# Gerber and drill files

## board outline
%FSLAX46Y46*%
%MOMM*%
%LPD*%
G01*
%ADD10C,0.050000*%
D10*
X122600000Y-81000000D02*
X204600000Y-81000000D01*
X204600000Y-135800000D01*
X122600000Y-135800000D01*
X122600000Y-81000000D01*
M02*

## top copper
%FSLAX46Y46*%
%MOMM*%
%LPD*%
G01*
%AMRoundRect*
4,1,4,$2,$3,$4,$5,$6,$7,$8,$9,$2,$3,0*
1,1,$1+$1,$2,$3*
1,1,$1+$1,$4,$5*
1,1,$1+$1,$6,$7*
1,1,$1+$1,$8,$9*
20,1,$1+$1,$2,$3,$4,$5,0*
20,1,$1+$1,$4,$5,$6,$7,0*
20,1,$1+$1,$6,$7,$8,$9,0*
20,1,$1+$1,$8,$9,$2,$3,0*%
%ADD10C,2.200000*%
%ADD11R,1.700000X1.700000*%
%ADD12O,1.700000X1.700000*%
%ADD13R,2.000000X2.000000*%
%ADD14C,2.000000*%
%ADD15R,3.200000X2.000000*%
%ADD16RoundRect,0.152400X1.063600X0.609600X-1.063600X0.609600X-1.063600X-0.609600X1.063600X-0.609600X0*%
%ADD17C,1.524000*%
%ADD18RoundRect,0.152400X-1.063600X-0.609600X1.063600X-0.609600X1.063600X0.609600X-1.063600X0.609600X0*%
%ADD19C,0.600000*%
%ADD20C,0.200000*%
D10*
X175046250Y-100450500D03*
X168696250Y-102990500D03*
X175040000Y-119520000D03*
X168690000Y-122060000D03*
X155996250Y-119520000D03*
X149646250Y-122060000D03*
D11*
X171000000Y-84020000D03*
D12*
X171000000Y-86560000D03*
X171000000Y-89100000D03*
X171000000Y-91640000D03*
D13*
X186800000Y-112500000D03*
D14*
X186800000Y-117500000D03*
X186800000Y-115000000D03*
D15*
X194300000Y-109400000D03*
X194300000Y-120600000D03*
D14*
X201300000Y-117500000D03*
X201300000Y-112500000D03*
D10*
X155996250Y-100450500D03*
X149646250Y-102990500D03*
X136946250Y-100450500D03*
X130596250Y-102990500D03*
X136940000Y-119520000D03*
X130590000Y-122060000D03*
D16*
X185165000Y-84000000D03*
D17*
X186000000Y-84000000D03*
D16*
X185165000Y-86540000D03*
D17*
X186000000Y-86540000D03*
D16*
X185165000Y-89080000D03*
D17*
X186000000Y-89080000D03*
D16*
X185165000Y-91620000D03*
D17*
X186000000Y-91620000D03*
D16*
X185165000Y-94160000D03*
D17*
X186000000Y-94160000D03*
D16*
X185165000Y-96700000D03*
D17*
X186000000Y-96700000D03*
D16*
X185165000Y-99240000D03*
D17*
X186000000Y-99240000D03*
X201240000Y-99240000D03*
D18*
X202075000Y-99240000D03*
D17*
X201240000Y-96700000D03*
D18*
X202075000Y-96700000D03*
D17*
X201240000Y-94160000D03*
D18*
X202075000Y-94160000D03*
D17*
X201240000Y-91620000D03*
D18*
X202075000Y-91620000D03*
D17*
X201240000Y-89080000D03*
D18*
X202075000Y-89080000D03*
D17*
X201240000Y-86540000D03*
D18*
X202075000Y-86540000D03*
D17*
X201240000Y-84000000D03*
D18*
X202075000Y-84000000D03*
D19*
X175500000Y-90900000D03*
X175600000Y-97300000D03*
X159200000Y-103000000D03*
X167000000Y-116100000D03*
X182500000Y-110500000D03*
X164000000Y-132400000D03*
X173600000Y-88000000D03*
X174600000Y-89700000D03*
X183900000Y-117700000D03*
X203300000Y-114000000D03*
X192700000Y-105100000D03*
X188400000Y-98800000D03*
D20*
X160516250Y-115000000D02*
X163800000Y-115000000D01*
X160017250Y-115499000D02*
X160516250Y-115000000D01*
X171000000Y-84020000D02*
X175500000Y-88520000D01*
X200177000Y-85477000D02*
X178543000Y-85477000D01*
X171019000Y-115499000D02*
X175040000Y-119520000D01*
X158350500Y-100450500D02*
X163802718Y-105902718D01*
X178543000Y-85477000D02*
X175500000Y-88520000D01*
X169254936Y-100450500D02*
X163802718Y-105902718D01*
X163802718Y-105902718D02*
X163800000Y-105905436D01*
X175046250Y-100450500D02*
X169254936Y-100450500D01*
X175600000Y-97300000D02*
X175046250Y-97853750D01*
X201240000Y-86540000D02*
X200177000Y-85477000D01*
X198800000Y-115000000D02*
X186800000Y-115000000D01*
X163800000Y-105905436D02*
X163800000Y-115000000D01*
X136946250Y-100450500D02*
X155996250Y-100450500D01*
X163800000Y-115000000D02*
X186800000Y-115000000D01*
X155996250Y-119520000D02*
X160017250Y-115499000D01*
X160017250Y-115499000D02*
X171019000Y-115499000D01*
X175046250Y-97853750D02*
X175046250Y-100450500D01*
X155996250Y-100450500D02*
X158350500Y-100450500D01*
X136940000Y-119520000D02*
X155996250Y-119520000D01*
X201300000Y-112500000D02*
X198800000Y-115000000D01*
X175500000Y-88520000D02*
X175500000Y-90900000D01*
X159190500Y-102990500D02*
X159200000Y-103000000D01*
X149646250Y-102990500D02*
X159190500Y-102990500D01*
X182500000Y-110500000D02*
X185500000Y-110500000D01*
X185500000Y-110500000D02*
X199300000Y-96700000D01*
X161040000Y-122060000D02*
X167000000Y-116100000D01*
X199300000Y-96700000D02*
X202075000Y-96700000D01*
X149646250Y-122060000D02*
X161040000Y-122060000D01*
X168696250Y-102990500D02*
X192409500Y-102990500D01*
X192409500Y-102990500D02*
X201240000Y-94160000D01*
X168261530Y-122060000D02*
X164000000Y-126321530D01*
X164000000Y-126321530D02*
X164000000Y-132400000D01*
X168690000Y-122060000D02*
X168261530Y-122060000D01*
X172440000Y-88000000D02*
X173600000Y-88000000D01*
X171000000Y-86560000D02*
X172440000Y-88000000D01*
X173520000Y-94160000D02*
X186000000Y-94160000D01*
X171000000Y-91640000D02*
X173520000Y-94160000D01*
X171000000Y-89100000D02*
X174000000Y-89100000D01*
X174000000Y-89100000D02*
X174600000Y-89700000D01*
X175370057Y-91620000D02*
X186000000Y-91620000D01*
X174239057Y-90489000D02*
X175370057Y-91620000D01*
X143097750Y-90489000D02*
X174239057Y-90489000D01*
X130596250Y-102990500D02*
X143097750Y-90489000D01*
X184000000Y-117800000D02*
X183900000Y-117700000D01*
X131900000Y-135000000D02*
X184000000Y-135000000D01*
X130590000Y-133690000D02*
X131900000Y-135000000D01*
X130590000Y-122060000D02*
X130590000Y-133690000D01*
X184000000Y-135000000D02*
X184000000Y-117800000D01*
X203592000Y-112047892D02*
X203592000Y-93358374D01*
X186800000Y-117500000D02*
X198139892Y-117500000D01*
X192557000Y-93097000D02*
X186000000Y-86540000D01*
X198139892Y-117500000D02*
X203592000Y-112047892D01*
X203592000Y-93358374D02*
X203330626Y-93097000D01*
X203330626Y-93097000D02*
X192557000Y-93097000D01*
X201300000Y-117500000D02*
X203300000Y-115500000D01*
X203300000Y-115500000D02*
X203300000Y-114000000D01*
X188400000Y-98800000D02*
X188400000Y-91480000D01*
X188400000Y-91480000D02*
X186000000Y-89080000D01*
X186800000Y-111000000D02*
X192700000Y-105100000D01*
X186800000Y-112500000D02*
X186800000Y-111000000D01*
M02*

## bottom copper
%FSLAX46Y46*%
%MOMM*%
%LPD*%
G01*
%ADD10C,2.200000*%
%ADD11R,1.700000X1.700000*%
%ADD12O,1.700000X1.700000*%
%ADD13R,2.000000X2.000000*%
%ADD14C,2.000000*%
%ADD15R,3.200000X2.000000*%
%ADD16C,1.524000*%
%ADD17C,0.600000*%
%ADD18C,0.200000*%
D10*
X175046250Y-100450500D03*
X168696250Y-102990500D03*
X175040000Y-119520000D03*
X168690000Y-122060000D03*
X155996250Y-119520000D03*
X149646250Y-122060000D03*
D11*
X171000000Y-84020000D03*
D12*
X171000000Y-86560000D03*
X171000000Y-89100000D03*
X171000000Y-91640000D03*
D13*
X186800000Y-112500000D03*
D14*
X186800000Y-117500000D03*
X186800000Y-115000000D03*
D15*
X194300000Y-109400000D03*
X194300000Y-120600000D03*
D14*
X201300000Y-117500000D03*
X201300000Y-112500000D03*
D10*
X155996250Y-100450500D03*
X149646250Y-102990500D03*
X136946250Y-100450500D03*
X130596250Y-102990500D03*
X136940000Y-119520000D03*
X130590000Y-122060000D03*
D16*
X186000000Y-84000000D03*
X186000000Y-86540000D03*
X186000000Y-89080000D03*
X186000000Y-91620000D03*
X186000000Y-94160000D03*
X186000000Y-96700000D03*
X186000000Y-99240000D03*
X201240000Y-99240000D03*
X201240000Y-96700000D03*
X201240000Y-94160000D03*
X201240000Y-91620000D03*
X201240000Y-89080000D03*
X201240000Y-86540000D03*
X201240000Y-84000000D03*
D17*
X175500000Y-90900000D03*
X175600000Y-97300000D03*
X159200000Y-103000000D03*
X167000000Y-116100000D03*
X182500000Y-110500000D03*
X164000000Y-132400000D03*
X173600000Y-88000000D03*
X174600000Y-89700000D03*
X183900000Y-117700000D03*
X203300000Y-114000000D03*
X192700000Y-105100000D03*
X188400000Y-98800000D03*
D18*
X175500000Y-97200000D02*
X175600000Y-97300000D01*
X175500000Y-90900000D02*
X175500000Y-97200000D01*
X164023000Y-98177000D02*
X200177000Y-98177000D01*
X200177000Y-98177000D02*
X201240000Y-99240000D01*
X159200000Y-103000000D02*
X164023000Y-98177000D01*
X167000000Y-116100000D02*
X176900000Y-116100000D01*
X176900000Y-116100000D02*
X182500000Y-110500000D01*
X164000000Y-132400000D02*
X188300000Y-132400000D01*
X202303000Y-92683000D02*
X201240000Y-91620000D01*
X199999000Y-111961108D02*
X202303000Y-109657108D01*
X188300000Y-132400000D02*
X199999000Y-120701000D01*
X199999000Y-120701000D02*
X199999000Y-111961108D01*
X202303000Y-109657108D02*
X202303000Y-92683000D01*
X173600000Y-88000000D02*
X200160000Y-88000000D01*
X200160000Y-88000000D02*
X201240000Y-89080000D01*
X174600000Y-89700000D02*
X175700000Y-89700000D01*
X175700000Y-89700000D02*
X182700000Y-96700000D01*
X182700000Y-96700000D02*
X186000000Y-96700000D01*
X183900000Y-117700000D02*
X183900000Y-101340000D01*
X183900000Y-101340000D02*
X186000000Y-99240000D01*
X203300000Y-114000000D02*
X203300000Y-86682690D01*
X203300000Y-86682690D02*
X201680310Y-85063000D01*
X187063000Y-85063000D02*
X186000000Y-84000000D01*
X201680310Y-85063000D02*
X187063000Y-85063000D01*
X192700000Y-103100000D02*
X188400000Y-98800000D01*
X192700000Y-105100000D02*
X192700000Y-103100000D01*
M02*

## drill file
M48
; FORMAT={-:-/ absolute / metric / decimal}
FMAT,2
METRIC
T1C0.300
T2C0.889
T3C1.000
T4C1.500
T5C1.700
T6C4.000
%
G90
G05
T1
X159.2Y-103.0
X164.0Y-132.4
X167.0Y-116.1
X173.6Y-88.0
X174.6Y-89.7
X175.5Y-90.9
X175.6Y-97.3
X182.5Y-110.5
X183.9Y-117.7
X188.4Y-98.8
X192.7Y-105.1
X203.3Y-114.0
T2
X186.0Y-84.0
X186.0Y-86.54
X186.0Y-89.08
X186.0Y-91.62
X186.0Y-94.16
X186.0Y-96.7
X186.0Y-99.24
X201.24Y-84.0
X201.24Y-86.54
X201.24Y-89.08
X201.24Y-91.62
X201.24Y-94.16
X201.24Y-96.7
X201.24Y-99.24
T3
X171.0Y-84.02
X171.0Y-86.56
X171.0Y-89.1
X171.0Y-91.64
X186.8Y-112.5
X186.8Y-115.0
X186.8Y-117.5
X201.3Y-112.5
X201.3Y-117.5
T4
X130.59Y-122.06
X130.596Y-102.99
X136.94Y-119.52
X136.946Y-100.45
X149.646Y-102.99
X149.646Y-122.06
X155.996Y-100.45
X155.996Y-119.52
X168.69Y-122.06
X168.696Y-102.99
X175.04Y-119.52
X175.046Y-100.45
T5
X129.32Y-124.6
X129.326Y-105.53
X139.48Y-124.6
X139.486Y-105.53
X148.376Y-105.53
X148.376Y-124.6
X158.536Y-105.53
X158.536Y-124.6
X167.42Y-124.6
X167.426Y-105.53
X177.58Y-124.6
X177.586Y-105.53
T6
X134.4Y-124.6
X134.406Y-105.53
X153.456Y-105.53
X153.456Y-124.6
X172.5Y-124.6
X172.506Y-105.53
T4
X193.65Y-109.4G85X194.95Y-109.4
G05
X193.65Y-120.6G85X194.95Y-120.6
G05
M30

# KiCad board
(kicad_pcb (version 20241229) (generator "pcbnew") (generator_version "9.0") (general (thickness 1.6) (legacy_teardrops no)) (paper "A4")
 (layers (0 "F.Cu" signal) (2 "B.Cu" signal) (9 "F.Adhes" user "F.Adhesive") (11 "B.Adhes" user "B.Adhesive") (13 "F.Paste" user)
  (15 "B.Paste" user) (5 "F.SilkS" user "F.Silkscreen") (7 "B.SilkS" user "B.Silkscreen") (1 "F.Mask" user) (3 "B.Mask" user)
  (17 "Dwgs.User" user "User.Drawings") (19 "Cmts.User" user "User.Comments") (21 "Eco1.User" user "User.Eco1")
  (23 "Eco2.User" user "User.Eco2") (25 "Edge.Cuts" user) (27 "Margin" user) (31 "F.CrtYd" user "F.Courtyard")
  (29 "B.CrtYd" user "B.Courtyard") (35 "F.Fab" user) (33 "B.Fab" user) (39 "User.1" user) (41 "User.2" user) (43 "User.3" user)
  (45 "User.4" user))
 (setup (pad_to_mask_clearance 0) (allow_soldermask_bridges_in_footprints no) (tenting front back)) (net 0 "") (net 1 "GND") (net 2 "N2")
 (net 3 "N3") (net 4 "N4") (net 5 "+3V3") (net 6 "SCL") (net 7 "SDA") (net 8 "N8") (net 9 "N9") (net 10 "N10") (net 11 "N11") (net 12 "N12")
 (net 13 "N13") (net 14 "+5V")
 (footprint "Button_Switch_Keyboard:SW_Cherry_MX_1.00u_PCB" (layer "F.Cu") (at 175.04625 100.4505)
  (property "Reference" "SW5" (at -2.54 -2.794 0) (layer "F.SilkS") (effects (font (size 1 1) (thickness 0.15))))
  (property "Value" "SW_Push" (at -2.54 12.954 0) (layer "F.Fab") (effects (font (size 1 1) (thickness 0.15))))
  (pad "" np_thru_hole circle (at -7.62 5.08) (size 1.7 1.7) (drill 1.7) (layers "*.Cu" "*.Mask"))
  (pad "" np_thru_hole circle (at -2.54 5.08) (size 4 4) (drill 4) (layers "*.Cu" "*.Mask"))
  (pad "" np_thru_hole circle (at 2.54 5.08) (size 1.7 1.7) (drill 1.7) (layers "*.Cu" "*.Mask"))
  (pad "1" thru_hole circle (at 0 0) (size 2.2 2.2) (drill 1.5) (layers "*.Cu" "*.Mask") (remove_unused_layers no) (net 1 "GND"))
  (pad "2" thru_hole circle (at -6.35 2.54) (size 2.2 2.2) (drill 1.5) (layers "*.Cu" "*.Mask") (remove_unused_layers no) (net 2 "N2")))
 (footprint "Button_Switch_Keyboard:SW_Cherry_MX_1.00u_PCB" (layer "F.Cu") (at 175.04 119.52)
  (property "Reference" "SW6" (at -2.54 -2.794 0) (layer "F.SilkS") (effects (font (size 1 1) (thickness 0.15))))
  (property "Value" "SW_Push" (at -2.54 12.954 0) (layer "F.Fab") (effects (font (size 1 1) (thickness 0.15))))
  (pad "" np_thru_hole circle (at -7.62 5.08) (size 1.7 1.7) (drill 1.7) (layers "*.Cu" "*.Mask"))
  (pad "" np_thru_hole circle (at -2.54 5.08) (size 4 4) (drill 4) (layers "*.Cu" "*.Mask"))
  (pad "" np_thru_hole circle (at 2.54 5.08) (size 1.7 1.7) (drill 1.7) (layers "*.Cu" "*.Mask"))
  (pad "1" thru_hole circle (at 0 0) (size 2.2 2.2) (drill 1.5) (layers "*.Cu" "*.Mask") (remove_unused_layers no) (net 1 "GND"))
  (pad "2" thru_hole circle (at -6.35 2.54) (size 2.2 2.2) (drill 1.5) (layers "*.Cu" "*.Mask") (remove_unused_layers no) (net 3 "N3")))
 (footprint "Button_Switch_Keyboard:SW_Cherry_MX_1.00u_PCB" (layer "F.Cu") (at 155.99625 119.52)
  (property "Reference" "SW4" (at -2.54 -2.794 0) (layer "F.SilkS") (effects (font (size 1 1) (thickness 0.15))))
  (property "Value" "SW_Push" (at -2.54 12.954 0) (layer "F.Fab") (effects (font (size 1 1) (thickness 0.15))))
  (pad "" np_thru_hole circle (at -7.62 5.08) (size 1.7 1.7) (drill 1.7) (layers "*.Cu" "*.Mask"))
  (pad "" np_thru_hole circle (at -2.54 5.08) (size 4 4) (drill 4) (layers "*.Cu" "*.Mask"))
  (pad "" np_thru_hole circle (at 2.54 5.08) (size 1.7 1.7) (drill 1.7) (layers "*.Cu" "*.Mask"))
  (pad "1" thru_hole circle (at 0 0) (size 2.2 2.2) (drill 1.5) (layers "*.Cu" "*.Mask") (remove_unused_layers no) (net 1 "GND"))
  (pad "2" thru_hole circle (at -6.35 2.54) (size 2.2 2.2) (drill 1.5) (layers "*.Cu" "*.Mask") (remove_unused_layers no) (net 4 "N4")))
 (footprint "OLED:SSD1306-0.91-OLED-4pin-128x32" (layer "F.Cu") (at 134.5 81.83)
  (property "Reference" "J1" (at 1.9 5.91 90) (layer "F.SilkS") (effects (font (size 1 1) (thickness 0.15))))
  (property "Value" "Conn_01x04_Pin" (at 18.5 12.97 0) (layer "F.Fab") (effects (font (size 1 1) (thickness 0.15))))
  (pad "1" thru_hole rect (at 36.5 2.19) (size 1.7 1.7) (drill 1) (layers "*.Cu" "*.Mask") (remove_unused_layers no) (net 1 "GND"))
  (pad "2" thru_hole oval (at 36.5 4.73) (size 1.7 1.7) (drill 1) (layers "*.Cu" "*.Mask") (remove_unused_layers no) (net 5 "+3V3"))
  (pad "3" thru_hole oval (at 36.5 7.27) (size 1.7 1.7) (drill 1) (layers "*.Cu" "*.Mask") (remove_unused_layers no) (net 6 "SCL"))
  (pad "4" thru_hole oval (at 36.5 9.81) (size 1.7 1.7) (drill 1) (layers "*.Cu" "*.Mask") (remove_unused_layers no) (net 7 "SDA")))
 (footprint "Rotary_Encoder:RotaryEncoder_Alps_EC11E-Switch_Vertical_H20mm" (layer "F.Cu") (at 186.8 112.5)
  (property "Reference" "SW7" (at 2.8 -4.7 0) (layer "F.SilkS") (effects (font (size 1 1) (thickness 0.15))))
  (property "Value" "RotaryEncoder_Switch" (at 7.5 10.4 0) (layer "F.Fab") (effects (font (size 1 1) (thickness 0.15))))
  (pad "A" thru_hole rect (at 0 0) (size 2 2) (drill 1) (layers "*.Cu" "*.Mask") (remove_unused_layers no) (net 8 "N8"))
  (pad "B" thru_hole circle (at 0 5) (size 2 2) (drill 1) (layers "*.Cu" "*.Mask") (remove_unused_layers no) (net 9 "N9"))
  (pad "C" thru_hole circle (at 0 2.5) (size 2 2) (drill 1) (layers "*.Cu" "*.Mask") (remove_unused_layers no) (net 1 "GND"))
  (pad "MP" thru_hole rect (at 7.5 -3.1) (size 3.2 2) (drill oval 2.8 1.5) (layers "*.Cu" "*.Mask") (remove_unused_layers no))
  (pad "MP" thru_hole rect (at 7.5 8.1) (size 3.2 2) (drill oval 2.8 1.5) (layers "*.Cu" "*.Mask") (remove_unused_layers no))
  (pad "S1" thru_hole circle (at 14.5 5) (size 2 2) (drill 1) (layers "*.Cu" "*.Mask") (remove_unused_layers no) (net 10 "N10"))
  (pad "S2" thru_hole circle (at 14.5 0) (size 2 2) (drill 1) (layers "*.Cu" "*.Mask") (remove_unused_layers no) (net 1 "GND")))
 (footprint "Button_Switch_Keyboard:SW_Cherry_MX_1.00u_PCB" (layer "F.Cu") (at 155.99625 100.4505)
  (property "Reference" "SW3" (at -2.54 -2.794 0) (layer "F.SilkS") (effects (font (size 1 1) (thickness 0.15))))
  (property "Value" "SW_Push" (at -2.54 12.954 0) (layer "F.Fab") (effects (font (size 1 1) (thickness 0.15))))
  (pad "" np_thru_hole circle (at -7.62 5.08) (size 1.7 1.7) (drill 1.7) (layers "*.Cu" "*.Mask"))
  (pad "" np_thru_hole circle (at -2.54 5.08) (size 4 4) (drill 4) (layers "*.Cu" "*.Mask"))
  (pad "" np_thru_hole circle (at 2.54 5.08) (size 1.7 1.7) (drill 1.7) (layers "*.Cu" "*.Mask"))
  (pad "1" thru_hole circle (at 0 0) (size 2.2 2.2) (drill 1.5) (layers "*.Cu" "*.Mask") (remove_unused_layers no) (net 1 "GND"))
  (pad "2" thru_hole circle (at -6.35 2.54) (size 2.2 2.2) (drill 1.5) (layers "*.Cu" "*.Mask") (remove_unused_layers no) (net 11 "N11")))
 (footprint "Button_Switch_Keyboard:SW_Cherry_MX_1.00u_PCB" (layer "F.Cu") (at 136.94625 100.4505)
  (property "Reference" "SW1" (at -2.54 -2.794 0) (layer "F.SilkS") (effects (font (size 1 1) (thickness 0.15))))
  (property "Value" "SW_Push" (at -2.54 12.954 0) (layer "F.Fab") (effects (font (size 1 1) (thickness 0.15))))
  (pad "" np_thru_hole circle (at -7.62 5.08) (size 1.7 1.7) (drill 1.7) (layers "*.Cu" "*.Mask"))
  (pad "" np_thru_hole circle (at -2.54 5.08) (size 4 4) (drill 4) (layers "*.Cu" "*.Mask"))
  (pad "" np_thru_hole circle (at 2.54 5.08) (size 1.7 1.7) (drill 1.7) (layers "*.Cu" "*.Mask"))
  (pad "1" thru_hole circle (at 0 0) (size 2.2 2.2) (drill 1.5) (layers "*.Cu" "*.Mask") (remove_unused_layers no) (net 1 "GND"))
  (pad "2" thru_hole circle (at -6.35 2.54) (size 2.2 2.2) (drill 1.5) (layers "*.Cu" "*.Mask") (remove_unused_layers no) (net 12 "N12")))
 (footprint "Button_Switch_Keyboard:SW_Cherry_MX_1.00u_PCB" (layer "F.Cu") (at 136.94 119.52)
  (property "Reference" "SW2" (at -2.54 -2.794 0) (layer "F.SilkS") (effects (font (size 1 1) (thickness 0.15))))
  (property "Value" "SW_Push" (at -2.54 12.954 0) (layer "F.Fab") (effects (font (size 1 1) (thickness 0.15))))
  (pad "" np_thru_hole circle (at -7.62 5.08) (size 1.7 1.7) (drill 1.7) (layers "*.Cu" "*.Mask"))
  (pad "" np_thru_hole circle (at -2.54 5.08) (size 4 4) (drill 4) (layers "*.Cu" "*.Mask"))
  (pad "" np_thru_hole circle (at 2.54 5.08) (size 1.7 1.7) (drill 1.7) (layers "*.Cu" "*.Mask"))
  (pad "1" thru_hole circle (at 0 0) (size 2.2 2.2) (drill 1.5) (layers "*.Cu" "*.Mask") (remove_unused_layers no) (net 1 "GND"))
  (pad "2" thru_hole circle (at -6.35 2.54) (size 2.2 2.2) (drill 1.5) (layers "*.Cu" "*.Mask") (remove_unused_layers no) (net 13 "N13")))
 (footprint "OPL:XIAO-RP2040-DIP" (layer "F.Cu") (at 193.62 91.62)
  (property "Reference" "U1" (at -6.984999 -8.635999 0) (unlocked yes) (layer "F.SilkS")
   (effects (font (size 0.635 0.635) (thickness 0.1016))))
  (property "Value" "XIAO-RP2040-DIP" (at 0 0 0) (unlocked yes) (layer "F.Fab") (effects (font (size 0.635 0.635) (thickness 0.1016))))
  (pad "1" smd roundrect (at -8.455 -7.62 180) (size 2.432 1.524) (layers "F.Cu" "F.Mask") (roundrect_rratio 0.1) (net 10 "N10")
   (thermal_bridge_angle 45))
  (pad "1" thru_hole circle (at -7.62 -7.62 180) (size 1.524 1.524) (drill 0.889) (layers "*.Cu" "*.Mask") (remove_unused_layers no)
   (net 10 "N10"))
  (pad "2" smd roundrect (at -8.455 -5.08 180) (size 2.432 1.524) (layers "F.Cu" "F.Mask") (roundrect_rratio 0.1) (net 9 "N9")
   (thermal_bridge_angle 45))
  (pad "2" thru_hole circle (at -7.62 -5.08 180) (size 1.524 1.524) (drill 0.889) (layers "*.Cu" "*.Mask") (remove_unused_layers no)
   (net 9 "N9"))
  (pad "3" smd roundrect (at -8.455 -2.54 180) (size 2.432 1.524) (layers "F.Cu" "F.Mask") (roundrect_rratio 0.1) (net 8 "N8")
   (thermal_bridge_angle 45))
  (pad "3" thru_hole circle (at -7.62 -2.54 180) (size 1.524 1.524) (drill 0.889) (layers "*.Cu" "*.Mask") (remove_unused_layers no)
   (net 8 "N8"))
  (pad "4" smd roundrect (at -8.455 0 180) (size 2.432 1.524) (layers "F.Cu" "F.Mask") (roundrect_rratio 0.1) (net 12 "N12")
   (thermal_bridge_angle 45))
  (pad "4" thru_hole circle (at -7.62 0 180) (size 1.524 1.524) (drill 0.889) (layers "*.Cu" "*.Mask") (remove_unused_layers no)
   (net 12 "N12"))
  (pad "5" smd roundrect (at -8.455 2.54 180) (size 2.432 1.524) (layers "F.Cu" "F.Mask") (roundrect_rratio 0.1) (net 7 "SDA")
   (thermal_bridge_angle 45))
  (pad "5" thru_hole circle (at -7.62 2.54 180) (size 1.524 1.524) (drill 0.889) (layers "*.Cu" "*.Mask") (remove_unused_layers no)
   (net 7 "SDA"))
  (pad "6" smd roundrect (at -8.455 5.08 180) (size 2.432 1.524) (layers "F.Cu" "F.Mask") (roundrect_rratio 0.1) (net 6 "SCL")
   (thermal_bridge_angle 45))
  (pad "6" thru_hole circle (at -7.62 5.08 180) (size 1.524 1.524) (drill 0.889) (layers "*.Cu" "*.Mask") (remove_unused_layers no)
   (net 6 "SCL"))
  (pad "7" smd roundrect (at -8.455 7.62 180) (size 2.432 1.524) (layers "F.Cu" "F.Mask") (roundrect_rratio 0.1) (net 13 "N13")
   (thermal_bridge_angle 45))
  (pad "7" thru_hole circle (at -7.62 7.62 180) (size 1.524 1.524) (drill 0.889) (layers "*.Cu" "*.Mask") (remove_unused_layers no)
   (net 13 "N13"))
  (pad "8" thru_hole circle (at 7.62 7.62) (size 1.524 1.524) (drill 0.889) (layers "*.Cu" "*.Mask") (remove_unused_layers no)
   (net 11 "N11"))
  (pad "8" smd roundrect (at 8.455 7.62) (size 2.432 1.524) (layers "F.Cu" "F.Mask") (roundrect_rratio 0.1) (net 11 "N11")
   (thermal_bridge_angle 45))
  (pad "9" thru_hole circle (at 7.62 5.08) (size 1.524 1.524) (drill 0.889) (layers "*.Cu" "*.Mask") (remove_unused_layers no) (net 4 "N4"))
  (pad "9" smd roundrect (at 8.455 5.08) (size 2.432 1.524) (layers "F.Cu" "F.Mask") (roundrect_rratio 0.1) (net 4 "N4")
   (thermal_bridge_angle 45))
  (pad "10" thru_hole circle (at 7.62 2.54) (size 1.524 1.524) (drill 0.889) (layers "*.Cu" "*.Mask") (remove_unused_layers no) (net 2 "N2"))
  (pad "10" smd roundrect (at 8.455 2.54) (size 2.432 1.524) (layers "F.Cu" "F.Mask") (roundrect_rratio 0.1) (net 2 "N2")
   (thermal_bridge_angle 45))
  (pad "11" thru_hole circle (at 7.62 0) (size 1.524 1.524) (drill 0.889) (layers "*.Cu" "*.Mask") (remove_unused_layers no) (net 3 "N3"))
  (pad "11" smd roundrect (at 8.455 0) (size 2.432 1.524) (layers "F.Cu" "F.Mask") (roundrect_rratio 0.1) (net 3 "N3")
   (thermal_bridge_angle 45))
  (pad "12" thru_hole circle (at 7.62 -2.54) (size 1.524 1.524) (drill 0.889) (layers "*.Cu" "*.Mask") (remove_unused_layers no)
   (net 5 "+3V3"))
  (pad "12" smd roundrect (at 8.455 -2.54) (size 2.432 1.524) (layers "F.Cu" "F.Mask") (roundrect_rratio 0.1) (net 5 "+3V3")
   (thermal_bridge_angle 45))
  (pad "13" thru_hole circle (at 7.62 -5.08) (size 1.524 1.524) (drill 0.889) (layers "*.Cu" "*.Mask") (remove_unused_layers no)
   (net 1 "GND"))
  (pad "13" smd roundrect (at 8.455 -5.08) (size 2.432 1.524) (layers "F.Cu" "F.Mask") (roundrect_rratio 0.1) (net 1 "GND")
   (thermal_bridge_angle 45))
  (pad "14" thru_hole circle (at 7.62 -7.62) (size 1.524 1.524) (drill 0.889) (layers "*.Cu" "*.Mask") (remove_unused_layers no)
   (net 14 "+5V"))
  (pad "14" smd roundrect (at 8.455 -7.62) (size 2.432 1.524) (layers "F.Cu" "F.Mask") (roundrect_rratio 0.1) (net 14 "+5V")
   (thermal_bridge_angle 45)))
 (gr_rect (start 122.6 81) (end 204.6 135.8) (stroke (width 0.05) (type default)) (fill no) (layer "Edge.Cuts"))
 (segment (start 160.51625 115) (end 163.8 115) (width 0.2) (layer "F.Cu") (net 1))
 (segment (start 160.01725 115.499) (end 160.51625 115) (width 0.2) (layer "F.Cu") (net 1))
 (segment (start 171 84.02) (end 175.5 88.52) (width 0.2) (layer "F.Cu") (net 1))
 (segment (start 200.177 85.477) (end 178.543 85.477) (width 0.2) (layer "F.Cu") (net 1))
 (segment (start 171.019 115.499) (end 175.04 119.52) (width 0.2) (layer "F.Cu") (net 1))
 (segment (start 158.3505 100.4505) (end 163.802718 105.902718) (width 0.2) (layer "F.Cu") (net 1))
 (segment (start 178.543 85.477) (end 175.5 88.52) (width 0.2) (layer "F.Cu") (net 1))
 (segment (start 169.254936 100.4505) (end 163.802718 105.902718) (width 0.2) (layer "F.Cu") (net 1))
 (segment (start 163.802718 105.902718) (end 163.8 105.905436) (width 0.2) (layer "F.Cu") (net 1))
 (segment (start 175.04625 100.4505) (end 169.254936 100.4505) (width 0.2) (layer "F.Cu") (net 1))
 (segment (start 175.6 97.3) (end 175.04625 97.85375) (width 0.2) (layer "F.Cu") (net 1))
 (segment (start 201.24 86.54) (end 200.177 85.477) (width 0.2) (layer "F.Cu") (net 1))
 (segment (start 198.8 115) (end 186.8 115) (width 0.2) (layer "F.Cu") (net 1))
 (segment (start 163.8 105.905436) (end 163.8 115) (width 0.2) (layer "F.Cu") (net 1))
 (segment (start 136.94625 100.4505) (end 155.99625 100.4505) (width 0.2) (layer "F.Cu") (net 1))
 (segment (start 163.8 115) (end 186.8 115) (width 0.2) (layer "F.Cu") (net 1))
 (segment (start 155.99625 119.52) (end 160.01725 115.499) (width 0.2) (layer "F.Cu") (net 1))
 (segment (start 160.01725 115.499) (end 171.019 115.499) (width 0.2) (layer "F.Cu") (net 1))
 (segment (start 175.04625 97.85375) (end 175.04625 100.4505) (width 0.2) (layer "F.Cu") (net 1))
 (segment (start 155.99625 100.4505) (end 158.3505 100.4505) (width 0.2) (layer "F.Cu") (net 1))
 (segment (start 136.94 119.52) (end 155.99625 119.52) (width 0.2) (layer "F.Cu") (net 1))
 (segment (start 201.3 112.5) (end 198.8 115) (width 0.2) (layer "F.Cu") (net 1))
 (segment (start 175.5 88.52) (end 175.5 90.9) (width 0.2) (layer "F.Cu") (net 1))
 (via (at 175.5 90.9) (size 0.6) (drill 0.3) (layers "F.Cu" "B.Cu") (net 1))
 (via (at 175.6 97.3) (size 0.6) (drill 0.3) (layers "F.Cu" "B.Cu") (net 1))
 (segment (start 175.5 97.2) (end 175.6 97.3) (width 0.2) (layer "B.Cu") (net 1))
 (segment (start 175.5 90.9) (end 175.5 97.2) (width 0.2) (layer "B.Cu") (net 1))
 (segment (start 159.1905 102.9905) (end 159.2 103) (width 0.2) (layer "F.Cu") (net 11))
 (segment (start 149.64625 102.9905) (end 159.1905 102.9905) (width 0.2) (layer "F.Cu") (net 11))
 (via (at 159.2 103) (size 0.6) (drill 0.3) (layers "F.Cu" "B.Cu") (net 11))
 (segment (start 164.023 98.177) (end 200.177 98.177) (width 0.2) (layer "B.Cu") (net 11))
 (segment (start 200.177 98.177) (end 201.24 99.24) (width 0.2) (layer "B.Cu") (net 11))
 (segment (start 159.2 103) (end 164.023 98.177) (width 0.2) (layer "B.Cu") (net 11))
 (segment (start 182.5 110.5) (end 185.5 110.5) (width 0.2) (layer "F.Cu") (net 4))
 (segment (start 185.5 110.5) (end 199.3 96.7) (width 0.2) (layer "F.Cu") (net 4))
 (segment (start 161.04 122.06) (end 167 116.1) (width 0.2) (layer "F.Cu") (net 4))
 (segment (start 199.3 96.7) (end 202.075 96.7) (width 0.2) (layer "F.Cu") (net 4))
 (segment (start 149.64625 122.06) (end 161.04 122.06) (width 0.2) (layer "F.Cu") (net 4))
 (via (at 167 116.1) (size 0.6) (drill 0.3) (layers "F.Cu" "B.Cu") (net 4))
 (via (at 182.5 110.5) (size 0.6) (drill 0.3) (layers "F.Cu" "B.Cu") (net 4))
 (segment (start 167 116.1) (end 176.9 116.1) (width 0.2) (layer "B.Cu") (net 4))
 (segment (start 176.9 116.1) (end 182.5 110.5) (width 0.2) (layer "B.Cu") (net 4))
 (segment (start 168.69625 102.9905) (end 192.4095 102.9905) (width 0.2) (layer "F.Cu") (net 2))
 (segment (start 192.4095 102.9905) (end 201.24 94.16) (width 0.2) (layer "F.Cu") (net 2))
 (segment (start 168.26153 122.06) (end 164 126.32153) (width 0.2) (layer "F.Cu") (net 3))
 (segment (start 164 126.32153) (end 164 132.4) (width 0.2) (layer "F.Cu") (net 3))
 (segment (start 168.69 122.06) (end 168.26153 122.06) (width 0.2) (layer "F.Cu") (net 3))
 (via (at 164 132.4) (size 0.6) (drill 0.3) (layers "F.Cu" "B.Cu") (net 3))
 (segment (start 164 132.4) (end 188.3 132.4) (width 0.2) (layer "B.Cu") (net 3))
 (segment (start 202.303 92.683) (end 201.24 91.62) (width 0.2) (layer "B.Cu") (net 3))
 (segment (start 199.999 111.961108) (end 202.303 109.657108) (width 0.2) (layer "B.Cu") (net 3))
 (segment (start 188.3 132.4) (end 199.999 120.701) (width 0.2) (layer "B.Cu") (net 3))
 (segment (start 199.999 120.701) (end 199.999 111.961108) (width 0.2) (layer "B.Cu") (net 3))
 (segment (start 202.303 109.657108) (end 202.303 92.683) (width 0.2) (layer "B.Cu") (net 3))
 (segment (start 172.44 88) (end 173.6 88) (width 0.2) (layer "F.Cu") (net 5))
 (segment (start 171 86.56) (end 172.44 88) (width 0.2) (layer "F.Cu") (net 5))
 (via (at 173.6 88) (size 0.6) (drill 0.3) (layers "F.Cu" "B.Cu") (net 5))
 (segment (start 173.6 88) (end 200.16 88) (width 0.2) (layer "B.Cu") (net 5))
 (segment (start 200.16 88) (end 201.24 89.08) (width 0.2) (layer "B.Cu") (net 5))
 (segment (start 173.52 94.16) (end 186 94.16) (width 0.2) (layer "F.Cu") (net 7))
 (segment (start 171 91.64) (end 173.52 94.16) (width 0.2) (layer "F.Cu") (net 7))
 (segment (start 171 89.1) (end 174 89.1) (width 0.2) (layer "F.Cu") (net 6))
 (segment (start 174 89.1) (end 174.6 89.7) (width 0.2) (layer "F.Cu") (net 6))
 (via (at 174.6 89.7) (size 0.6) (drill 0.3) (layers "F.Cu" "B.Cu") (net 6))
 (segment (start 174.6 89.7) (end 175.7 89.7) (width 0.2) (layer "B.Cu") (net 6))
 (segment (start 175.7 89.7) (end 182.7 96.7) (width 0.2) (layer "B.Cu") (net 6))
 (segment (start 182.7 96.7) (end 186 96.7) (width 0.2) (layer "B.Cu") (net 6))
 (segment (start 175.370057 91.62) (end 186 91.62) (width 0.2) (layer "F.Cu") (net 12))
 (segment (start 174.239057 90.489) (end 175.370057 91.62) (width 0.2) (layer "F.Cu") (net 12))
 (segment (start 143.09775 90.489) (end 174.239057 90.489) (width 0.2) (layer "F.Cu") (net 12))
 (segment (start 130.59625 102.9905) (end 143.09775 90.489) (width 0.2) (layer "F.Cu") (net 12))
 (segment (start 184 117.8) (end 183.9 117.7) (width 0.2) (layer "F.Cu") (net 13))
 (segment (start 131.9 135) (end 184 135) (width 0.2) (layer "F.Cu") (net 13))
 (segment (start 130.59 133.69) (end 131.9 135) (width 0.2) (layer "F.Cu") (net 13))
 (segment (start 130.59 122.06) (end 130.59 133.69) (width 0.2) (layer "F.Cu") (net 13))
 (segment (start 184 135) (end 184 117.8) (width 0.2) (layer "F.Cu") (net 13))
 (via (at 183.9 117.7) (size 0.6) (drill 0.3) (layers "F.Cu" "B.Cu") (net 13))
 (segment (start 183.9 117.7) (end 183.9 101.34) (width 0.2) (layer "B.Cu") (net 13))
 (segment (start 183.9 101.34) (end 186 99.24) (width 0.2) (layer "B.Cu") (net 13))
 (segment (start 203.592 112.047892) (end 203.592 93.358374) (width 0.2) (layer "F.Cu") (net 9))
 (segment (start 186.8 117.5) (end 198.139892 117.5) (width 0.2) (layer "F.Cu") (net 9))
 (segment (start 192.557 93.097) (end 186 86.54) (width 0.2) (layer "F.Cu") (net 9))
 (segment (start 198.139892 117.5) (end 203.592 112.047892) (width 0.2) (layer "F.Cu") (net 9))
 (segment (start 203.592 93.358374) (end 203.330626 93.097) (width 0.2) (layer "F.Cu") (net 9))
 (segment (start 203.330626 93.097) (end 192.557 93.097) (width 0.2) (layer "F.Cu") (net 9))
 (segment (start 201.3 117.5) (end 203.3 115.5) (width 0.2) (layer "F.Cu") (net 10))
 (segment (start 203.3 115.5) (end 203.3 114) (width 0.2) (layer "F.Cu") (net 10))
 (via (at 203.3 114) (size 0.6) (drill 0.3) (layers "F.Cu" "B.Cu") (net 10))
 (segment (start 203.3 114) (end 203.3 86.68269) (width 0.2) (layer "B.Cu") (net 10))
 (segment (start 203.3 86.68269) (end 201.68031 85.063) (width 0.2) (layer "B.Cu") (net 10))
 (segment (start 187.063 85.063) (end 186 84) (width 0.2) (layer "B.Cu") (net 10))
 (segment (start 201.68031 85.063) (end 187.063 85.063) (width 0.2) (layer "B.Cu") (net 10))
 (segment (start 188.4 98.8) (end 188.4 91.48) (width 0.2) (layer "F.Cu") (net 8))
 (segment (start 188.4 91.48) (end 186 89.08) (width 0.2) (layer "F.Cu") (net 8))
 (segment (start 186.8 111) (end 192.7 105.1) (width 0.2) (layer "F.Cu") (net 8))
 (segment (start 186.8 112.5) (end 186.8 111) (width 0.2) (layer "F.Cu") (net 8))
 (via (at 192.7 105.1) (size 0.6) (drill 0.3) (layers "F.Cu" "B.Cu") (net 8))
 (via (at 188.4 98.8) (size 0.6) (drill 0.3) (layers "F.Cu" "B.Cu") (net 8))
 (segment (start 192.7 103.1) (end 188.4 98.8) (width 0.2) (layer "B.Cu") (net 8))
 (segment (start 192.7 105.1) (end 192.7 103.1) (width 0.2) (layer "B.Cu") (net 8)))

